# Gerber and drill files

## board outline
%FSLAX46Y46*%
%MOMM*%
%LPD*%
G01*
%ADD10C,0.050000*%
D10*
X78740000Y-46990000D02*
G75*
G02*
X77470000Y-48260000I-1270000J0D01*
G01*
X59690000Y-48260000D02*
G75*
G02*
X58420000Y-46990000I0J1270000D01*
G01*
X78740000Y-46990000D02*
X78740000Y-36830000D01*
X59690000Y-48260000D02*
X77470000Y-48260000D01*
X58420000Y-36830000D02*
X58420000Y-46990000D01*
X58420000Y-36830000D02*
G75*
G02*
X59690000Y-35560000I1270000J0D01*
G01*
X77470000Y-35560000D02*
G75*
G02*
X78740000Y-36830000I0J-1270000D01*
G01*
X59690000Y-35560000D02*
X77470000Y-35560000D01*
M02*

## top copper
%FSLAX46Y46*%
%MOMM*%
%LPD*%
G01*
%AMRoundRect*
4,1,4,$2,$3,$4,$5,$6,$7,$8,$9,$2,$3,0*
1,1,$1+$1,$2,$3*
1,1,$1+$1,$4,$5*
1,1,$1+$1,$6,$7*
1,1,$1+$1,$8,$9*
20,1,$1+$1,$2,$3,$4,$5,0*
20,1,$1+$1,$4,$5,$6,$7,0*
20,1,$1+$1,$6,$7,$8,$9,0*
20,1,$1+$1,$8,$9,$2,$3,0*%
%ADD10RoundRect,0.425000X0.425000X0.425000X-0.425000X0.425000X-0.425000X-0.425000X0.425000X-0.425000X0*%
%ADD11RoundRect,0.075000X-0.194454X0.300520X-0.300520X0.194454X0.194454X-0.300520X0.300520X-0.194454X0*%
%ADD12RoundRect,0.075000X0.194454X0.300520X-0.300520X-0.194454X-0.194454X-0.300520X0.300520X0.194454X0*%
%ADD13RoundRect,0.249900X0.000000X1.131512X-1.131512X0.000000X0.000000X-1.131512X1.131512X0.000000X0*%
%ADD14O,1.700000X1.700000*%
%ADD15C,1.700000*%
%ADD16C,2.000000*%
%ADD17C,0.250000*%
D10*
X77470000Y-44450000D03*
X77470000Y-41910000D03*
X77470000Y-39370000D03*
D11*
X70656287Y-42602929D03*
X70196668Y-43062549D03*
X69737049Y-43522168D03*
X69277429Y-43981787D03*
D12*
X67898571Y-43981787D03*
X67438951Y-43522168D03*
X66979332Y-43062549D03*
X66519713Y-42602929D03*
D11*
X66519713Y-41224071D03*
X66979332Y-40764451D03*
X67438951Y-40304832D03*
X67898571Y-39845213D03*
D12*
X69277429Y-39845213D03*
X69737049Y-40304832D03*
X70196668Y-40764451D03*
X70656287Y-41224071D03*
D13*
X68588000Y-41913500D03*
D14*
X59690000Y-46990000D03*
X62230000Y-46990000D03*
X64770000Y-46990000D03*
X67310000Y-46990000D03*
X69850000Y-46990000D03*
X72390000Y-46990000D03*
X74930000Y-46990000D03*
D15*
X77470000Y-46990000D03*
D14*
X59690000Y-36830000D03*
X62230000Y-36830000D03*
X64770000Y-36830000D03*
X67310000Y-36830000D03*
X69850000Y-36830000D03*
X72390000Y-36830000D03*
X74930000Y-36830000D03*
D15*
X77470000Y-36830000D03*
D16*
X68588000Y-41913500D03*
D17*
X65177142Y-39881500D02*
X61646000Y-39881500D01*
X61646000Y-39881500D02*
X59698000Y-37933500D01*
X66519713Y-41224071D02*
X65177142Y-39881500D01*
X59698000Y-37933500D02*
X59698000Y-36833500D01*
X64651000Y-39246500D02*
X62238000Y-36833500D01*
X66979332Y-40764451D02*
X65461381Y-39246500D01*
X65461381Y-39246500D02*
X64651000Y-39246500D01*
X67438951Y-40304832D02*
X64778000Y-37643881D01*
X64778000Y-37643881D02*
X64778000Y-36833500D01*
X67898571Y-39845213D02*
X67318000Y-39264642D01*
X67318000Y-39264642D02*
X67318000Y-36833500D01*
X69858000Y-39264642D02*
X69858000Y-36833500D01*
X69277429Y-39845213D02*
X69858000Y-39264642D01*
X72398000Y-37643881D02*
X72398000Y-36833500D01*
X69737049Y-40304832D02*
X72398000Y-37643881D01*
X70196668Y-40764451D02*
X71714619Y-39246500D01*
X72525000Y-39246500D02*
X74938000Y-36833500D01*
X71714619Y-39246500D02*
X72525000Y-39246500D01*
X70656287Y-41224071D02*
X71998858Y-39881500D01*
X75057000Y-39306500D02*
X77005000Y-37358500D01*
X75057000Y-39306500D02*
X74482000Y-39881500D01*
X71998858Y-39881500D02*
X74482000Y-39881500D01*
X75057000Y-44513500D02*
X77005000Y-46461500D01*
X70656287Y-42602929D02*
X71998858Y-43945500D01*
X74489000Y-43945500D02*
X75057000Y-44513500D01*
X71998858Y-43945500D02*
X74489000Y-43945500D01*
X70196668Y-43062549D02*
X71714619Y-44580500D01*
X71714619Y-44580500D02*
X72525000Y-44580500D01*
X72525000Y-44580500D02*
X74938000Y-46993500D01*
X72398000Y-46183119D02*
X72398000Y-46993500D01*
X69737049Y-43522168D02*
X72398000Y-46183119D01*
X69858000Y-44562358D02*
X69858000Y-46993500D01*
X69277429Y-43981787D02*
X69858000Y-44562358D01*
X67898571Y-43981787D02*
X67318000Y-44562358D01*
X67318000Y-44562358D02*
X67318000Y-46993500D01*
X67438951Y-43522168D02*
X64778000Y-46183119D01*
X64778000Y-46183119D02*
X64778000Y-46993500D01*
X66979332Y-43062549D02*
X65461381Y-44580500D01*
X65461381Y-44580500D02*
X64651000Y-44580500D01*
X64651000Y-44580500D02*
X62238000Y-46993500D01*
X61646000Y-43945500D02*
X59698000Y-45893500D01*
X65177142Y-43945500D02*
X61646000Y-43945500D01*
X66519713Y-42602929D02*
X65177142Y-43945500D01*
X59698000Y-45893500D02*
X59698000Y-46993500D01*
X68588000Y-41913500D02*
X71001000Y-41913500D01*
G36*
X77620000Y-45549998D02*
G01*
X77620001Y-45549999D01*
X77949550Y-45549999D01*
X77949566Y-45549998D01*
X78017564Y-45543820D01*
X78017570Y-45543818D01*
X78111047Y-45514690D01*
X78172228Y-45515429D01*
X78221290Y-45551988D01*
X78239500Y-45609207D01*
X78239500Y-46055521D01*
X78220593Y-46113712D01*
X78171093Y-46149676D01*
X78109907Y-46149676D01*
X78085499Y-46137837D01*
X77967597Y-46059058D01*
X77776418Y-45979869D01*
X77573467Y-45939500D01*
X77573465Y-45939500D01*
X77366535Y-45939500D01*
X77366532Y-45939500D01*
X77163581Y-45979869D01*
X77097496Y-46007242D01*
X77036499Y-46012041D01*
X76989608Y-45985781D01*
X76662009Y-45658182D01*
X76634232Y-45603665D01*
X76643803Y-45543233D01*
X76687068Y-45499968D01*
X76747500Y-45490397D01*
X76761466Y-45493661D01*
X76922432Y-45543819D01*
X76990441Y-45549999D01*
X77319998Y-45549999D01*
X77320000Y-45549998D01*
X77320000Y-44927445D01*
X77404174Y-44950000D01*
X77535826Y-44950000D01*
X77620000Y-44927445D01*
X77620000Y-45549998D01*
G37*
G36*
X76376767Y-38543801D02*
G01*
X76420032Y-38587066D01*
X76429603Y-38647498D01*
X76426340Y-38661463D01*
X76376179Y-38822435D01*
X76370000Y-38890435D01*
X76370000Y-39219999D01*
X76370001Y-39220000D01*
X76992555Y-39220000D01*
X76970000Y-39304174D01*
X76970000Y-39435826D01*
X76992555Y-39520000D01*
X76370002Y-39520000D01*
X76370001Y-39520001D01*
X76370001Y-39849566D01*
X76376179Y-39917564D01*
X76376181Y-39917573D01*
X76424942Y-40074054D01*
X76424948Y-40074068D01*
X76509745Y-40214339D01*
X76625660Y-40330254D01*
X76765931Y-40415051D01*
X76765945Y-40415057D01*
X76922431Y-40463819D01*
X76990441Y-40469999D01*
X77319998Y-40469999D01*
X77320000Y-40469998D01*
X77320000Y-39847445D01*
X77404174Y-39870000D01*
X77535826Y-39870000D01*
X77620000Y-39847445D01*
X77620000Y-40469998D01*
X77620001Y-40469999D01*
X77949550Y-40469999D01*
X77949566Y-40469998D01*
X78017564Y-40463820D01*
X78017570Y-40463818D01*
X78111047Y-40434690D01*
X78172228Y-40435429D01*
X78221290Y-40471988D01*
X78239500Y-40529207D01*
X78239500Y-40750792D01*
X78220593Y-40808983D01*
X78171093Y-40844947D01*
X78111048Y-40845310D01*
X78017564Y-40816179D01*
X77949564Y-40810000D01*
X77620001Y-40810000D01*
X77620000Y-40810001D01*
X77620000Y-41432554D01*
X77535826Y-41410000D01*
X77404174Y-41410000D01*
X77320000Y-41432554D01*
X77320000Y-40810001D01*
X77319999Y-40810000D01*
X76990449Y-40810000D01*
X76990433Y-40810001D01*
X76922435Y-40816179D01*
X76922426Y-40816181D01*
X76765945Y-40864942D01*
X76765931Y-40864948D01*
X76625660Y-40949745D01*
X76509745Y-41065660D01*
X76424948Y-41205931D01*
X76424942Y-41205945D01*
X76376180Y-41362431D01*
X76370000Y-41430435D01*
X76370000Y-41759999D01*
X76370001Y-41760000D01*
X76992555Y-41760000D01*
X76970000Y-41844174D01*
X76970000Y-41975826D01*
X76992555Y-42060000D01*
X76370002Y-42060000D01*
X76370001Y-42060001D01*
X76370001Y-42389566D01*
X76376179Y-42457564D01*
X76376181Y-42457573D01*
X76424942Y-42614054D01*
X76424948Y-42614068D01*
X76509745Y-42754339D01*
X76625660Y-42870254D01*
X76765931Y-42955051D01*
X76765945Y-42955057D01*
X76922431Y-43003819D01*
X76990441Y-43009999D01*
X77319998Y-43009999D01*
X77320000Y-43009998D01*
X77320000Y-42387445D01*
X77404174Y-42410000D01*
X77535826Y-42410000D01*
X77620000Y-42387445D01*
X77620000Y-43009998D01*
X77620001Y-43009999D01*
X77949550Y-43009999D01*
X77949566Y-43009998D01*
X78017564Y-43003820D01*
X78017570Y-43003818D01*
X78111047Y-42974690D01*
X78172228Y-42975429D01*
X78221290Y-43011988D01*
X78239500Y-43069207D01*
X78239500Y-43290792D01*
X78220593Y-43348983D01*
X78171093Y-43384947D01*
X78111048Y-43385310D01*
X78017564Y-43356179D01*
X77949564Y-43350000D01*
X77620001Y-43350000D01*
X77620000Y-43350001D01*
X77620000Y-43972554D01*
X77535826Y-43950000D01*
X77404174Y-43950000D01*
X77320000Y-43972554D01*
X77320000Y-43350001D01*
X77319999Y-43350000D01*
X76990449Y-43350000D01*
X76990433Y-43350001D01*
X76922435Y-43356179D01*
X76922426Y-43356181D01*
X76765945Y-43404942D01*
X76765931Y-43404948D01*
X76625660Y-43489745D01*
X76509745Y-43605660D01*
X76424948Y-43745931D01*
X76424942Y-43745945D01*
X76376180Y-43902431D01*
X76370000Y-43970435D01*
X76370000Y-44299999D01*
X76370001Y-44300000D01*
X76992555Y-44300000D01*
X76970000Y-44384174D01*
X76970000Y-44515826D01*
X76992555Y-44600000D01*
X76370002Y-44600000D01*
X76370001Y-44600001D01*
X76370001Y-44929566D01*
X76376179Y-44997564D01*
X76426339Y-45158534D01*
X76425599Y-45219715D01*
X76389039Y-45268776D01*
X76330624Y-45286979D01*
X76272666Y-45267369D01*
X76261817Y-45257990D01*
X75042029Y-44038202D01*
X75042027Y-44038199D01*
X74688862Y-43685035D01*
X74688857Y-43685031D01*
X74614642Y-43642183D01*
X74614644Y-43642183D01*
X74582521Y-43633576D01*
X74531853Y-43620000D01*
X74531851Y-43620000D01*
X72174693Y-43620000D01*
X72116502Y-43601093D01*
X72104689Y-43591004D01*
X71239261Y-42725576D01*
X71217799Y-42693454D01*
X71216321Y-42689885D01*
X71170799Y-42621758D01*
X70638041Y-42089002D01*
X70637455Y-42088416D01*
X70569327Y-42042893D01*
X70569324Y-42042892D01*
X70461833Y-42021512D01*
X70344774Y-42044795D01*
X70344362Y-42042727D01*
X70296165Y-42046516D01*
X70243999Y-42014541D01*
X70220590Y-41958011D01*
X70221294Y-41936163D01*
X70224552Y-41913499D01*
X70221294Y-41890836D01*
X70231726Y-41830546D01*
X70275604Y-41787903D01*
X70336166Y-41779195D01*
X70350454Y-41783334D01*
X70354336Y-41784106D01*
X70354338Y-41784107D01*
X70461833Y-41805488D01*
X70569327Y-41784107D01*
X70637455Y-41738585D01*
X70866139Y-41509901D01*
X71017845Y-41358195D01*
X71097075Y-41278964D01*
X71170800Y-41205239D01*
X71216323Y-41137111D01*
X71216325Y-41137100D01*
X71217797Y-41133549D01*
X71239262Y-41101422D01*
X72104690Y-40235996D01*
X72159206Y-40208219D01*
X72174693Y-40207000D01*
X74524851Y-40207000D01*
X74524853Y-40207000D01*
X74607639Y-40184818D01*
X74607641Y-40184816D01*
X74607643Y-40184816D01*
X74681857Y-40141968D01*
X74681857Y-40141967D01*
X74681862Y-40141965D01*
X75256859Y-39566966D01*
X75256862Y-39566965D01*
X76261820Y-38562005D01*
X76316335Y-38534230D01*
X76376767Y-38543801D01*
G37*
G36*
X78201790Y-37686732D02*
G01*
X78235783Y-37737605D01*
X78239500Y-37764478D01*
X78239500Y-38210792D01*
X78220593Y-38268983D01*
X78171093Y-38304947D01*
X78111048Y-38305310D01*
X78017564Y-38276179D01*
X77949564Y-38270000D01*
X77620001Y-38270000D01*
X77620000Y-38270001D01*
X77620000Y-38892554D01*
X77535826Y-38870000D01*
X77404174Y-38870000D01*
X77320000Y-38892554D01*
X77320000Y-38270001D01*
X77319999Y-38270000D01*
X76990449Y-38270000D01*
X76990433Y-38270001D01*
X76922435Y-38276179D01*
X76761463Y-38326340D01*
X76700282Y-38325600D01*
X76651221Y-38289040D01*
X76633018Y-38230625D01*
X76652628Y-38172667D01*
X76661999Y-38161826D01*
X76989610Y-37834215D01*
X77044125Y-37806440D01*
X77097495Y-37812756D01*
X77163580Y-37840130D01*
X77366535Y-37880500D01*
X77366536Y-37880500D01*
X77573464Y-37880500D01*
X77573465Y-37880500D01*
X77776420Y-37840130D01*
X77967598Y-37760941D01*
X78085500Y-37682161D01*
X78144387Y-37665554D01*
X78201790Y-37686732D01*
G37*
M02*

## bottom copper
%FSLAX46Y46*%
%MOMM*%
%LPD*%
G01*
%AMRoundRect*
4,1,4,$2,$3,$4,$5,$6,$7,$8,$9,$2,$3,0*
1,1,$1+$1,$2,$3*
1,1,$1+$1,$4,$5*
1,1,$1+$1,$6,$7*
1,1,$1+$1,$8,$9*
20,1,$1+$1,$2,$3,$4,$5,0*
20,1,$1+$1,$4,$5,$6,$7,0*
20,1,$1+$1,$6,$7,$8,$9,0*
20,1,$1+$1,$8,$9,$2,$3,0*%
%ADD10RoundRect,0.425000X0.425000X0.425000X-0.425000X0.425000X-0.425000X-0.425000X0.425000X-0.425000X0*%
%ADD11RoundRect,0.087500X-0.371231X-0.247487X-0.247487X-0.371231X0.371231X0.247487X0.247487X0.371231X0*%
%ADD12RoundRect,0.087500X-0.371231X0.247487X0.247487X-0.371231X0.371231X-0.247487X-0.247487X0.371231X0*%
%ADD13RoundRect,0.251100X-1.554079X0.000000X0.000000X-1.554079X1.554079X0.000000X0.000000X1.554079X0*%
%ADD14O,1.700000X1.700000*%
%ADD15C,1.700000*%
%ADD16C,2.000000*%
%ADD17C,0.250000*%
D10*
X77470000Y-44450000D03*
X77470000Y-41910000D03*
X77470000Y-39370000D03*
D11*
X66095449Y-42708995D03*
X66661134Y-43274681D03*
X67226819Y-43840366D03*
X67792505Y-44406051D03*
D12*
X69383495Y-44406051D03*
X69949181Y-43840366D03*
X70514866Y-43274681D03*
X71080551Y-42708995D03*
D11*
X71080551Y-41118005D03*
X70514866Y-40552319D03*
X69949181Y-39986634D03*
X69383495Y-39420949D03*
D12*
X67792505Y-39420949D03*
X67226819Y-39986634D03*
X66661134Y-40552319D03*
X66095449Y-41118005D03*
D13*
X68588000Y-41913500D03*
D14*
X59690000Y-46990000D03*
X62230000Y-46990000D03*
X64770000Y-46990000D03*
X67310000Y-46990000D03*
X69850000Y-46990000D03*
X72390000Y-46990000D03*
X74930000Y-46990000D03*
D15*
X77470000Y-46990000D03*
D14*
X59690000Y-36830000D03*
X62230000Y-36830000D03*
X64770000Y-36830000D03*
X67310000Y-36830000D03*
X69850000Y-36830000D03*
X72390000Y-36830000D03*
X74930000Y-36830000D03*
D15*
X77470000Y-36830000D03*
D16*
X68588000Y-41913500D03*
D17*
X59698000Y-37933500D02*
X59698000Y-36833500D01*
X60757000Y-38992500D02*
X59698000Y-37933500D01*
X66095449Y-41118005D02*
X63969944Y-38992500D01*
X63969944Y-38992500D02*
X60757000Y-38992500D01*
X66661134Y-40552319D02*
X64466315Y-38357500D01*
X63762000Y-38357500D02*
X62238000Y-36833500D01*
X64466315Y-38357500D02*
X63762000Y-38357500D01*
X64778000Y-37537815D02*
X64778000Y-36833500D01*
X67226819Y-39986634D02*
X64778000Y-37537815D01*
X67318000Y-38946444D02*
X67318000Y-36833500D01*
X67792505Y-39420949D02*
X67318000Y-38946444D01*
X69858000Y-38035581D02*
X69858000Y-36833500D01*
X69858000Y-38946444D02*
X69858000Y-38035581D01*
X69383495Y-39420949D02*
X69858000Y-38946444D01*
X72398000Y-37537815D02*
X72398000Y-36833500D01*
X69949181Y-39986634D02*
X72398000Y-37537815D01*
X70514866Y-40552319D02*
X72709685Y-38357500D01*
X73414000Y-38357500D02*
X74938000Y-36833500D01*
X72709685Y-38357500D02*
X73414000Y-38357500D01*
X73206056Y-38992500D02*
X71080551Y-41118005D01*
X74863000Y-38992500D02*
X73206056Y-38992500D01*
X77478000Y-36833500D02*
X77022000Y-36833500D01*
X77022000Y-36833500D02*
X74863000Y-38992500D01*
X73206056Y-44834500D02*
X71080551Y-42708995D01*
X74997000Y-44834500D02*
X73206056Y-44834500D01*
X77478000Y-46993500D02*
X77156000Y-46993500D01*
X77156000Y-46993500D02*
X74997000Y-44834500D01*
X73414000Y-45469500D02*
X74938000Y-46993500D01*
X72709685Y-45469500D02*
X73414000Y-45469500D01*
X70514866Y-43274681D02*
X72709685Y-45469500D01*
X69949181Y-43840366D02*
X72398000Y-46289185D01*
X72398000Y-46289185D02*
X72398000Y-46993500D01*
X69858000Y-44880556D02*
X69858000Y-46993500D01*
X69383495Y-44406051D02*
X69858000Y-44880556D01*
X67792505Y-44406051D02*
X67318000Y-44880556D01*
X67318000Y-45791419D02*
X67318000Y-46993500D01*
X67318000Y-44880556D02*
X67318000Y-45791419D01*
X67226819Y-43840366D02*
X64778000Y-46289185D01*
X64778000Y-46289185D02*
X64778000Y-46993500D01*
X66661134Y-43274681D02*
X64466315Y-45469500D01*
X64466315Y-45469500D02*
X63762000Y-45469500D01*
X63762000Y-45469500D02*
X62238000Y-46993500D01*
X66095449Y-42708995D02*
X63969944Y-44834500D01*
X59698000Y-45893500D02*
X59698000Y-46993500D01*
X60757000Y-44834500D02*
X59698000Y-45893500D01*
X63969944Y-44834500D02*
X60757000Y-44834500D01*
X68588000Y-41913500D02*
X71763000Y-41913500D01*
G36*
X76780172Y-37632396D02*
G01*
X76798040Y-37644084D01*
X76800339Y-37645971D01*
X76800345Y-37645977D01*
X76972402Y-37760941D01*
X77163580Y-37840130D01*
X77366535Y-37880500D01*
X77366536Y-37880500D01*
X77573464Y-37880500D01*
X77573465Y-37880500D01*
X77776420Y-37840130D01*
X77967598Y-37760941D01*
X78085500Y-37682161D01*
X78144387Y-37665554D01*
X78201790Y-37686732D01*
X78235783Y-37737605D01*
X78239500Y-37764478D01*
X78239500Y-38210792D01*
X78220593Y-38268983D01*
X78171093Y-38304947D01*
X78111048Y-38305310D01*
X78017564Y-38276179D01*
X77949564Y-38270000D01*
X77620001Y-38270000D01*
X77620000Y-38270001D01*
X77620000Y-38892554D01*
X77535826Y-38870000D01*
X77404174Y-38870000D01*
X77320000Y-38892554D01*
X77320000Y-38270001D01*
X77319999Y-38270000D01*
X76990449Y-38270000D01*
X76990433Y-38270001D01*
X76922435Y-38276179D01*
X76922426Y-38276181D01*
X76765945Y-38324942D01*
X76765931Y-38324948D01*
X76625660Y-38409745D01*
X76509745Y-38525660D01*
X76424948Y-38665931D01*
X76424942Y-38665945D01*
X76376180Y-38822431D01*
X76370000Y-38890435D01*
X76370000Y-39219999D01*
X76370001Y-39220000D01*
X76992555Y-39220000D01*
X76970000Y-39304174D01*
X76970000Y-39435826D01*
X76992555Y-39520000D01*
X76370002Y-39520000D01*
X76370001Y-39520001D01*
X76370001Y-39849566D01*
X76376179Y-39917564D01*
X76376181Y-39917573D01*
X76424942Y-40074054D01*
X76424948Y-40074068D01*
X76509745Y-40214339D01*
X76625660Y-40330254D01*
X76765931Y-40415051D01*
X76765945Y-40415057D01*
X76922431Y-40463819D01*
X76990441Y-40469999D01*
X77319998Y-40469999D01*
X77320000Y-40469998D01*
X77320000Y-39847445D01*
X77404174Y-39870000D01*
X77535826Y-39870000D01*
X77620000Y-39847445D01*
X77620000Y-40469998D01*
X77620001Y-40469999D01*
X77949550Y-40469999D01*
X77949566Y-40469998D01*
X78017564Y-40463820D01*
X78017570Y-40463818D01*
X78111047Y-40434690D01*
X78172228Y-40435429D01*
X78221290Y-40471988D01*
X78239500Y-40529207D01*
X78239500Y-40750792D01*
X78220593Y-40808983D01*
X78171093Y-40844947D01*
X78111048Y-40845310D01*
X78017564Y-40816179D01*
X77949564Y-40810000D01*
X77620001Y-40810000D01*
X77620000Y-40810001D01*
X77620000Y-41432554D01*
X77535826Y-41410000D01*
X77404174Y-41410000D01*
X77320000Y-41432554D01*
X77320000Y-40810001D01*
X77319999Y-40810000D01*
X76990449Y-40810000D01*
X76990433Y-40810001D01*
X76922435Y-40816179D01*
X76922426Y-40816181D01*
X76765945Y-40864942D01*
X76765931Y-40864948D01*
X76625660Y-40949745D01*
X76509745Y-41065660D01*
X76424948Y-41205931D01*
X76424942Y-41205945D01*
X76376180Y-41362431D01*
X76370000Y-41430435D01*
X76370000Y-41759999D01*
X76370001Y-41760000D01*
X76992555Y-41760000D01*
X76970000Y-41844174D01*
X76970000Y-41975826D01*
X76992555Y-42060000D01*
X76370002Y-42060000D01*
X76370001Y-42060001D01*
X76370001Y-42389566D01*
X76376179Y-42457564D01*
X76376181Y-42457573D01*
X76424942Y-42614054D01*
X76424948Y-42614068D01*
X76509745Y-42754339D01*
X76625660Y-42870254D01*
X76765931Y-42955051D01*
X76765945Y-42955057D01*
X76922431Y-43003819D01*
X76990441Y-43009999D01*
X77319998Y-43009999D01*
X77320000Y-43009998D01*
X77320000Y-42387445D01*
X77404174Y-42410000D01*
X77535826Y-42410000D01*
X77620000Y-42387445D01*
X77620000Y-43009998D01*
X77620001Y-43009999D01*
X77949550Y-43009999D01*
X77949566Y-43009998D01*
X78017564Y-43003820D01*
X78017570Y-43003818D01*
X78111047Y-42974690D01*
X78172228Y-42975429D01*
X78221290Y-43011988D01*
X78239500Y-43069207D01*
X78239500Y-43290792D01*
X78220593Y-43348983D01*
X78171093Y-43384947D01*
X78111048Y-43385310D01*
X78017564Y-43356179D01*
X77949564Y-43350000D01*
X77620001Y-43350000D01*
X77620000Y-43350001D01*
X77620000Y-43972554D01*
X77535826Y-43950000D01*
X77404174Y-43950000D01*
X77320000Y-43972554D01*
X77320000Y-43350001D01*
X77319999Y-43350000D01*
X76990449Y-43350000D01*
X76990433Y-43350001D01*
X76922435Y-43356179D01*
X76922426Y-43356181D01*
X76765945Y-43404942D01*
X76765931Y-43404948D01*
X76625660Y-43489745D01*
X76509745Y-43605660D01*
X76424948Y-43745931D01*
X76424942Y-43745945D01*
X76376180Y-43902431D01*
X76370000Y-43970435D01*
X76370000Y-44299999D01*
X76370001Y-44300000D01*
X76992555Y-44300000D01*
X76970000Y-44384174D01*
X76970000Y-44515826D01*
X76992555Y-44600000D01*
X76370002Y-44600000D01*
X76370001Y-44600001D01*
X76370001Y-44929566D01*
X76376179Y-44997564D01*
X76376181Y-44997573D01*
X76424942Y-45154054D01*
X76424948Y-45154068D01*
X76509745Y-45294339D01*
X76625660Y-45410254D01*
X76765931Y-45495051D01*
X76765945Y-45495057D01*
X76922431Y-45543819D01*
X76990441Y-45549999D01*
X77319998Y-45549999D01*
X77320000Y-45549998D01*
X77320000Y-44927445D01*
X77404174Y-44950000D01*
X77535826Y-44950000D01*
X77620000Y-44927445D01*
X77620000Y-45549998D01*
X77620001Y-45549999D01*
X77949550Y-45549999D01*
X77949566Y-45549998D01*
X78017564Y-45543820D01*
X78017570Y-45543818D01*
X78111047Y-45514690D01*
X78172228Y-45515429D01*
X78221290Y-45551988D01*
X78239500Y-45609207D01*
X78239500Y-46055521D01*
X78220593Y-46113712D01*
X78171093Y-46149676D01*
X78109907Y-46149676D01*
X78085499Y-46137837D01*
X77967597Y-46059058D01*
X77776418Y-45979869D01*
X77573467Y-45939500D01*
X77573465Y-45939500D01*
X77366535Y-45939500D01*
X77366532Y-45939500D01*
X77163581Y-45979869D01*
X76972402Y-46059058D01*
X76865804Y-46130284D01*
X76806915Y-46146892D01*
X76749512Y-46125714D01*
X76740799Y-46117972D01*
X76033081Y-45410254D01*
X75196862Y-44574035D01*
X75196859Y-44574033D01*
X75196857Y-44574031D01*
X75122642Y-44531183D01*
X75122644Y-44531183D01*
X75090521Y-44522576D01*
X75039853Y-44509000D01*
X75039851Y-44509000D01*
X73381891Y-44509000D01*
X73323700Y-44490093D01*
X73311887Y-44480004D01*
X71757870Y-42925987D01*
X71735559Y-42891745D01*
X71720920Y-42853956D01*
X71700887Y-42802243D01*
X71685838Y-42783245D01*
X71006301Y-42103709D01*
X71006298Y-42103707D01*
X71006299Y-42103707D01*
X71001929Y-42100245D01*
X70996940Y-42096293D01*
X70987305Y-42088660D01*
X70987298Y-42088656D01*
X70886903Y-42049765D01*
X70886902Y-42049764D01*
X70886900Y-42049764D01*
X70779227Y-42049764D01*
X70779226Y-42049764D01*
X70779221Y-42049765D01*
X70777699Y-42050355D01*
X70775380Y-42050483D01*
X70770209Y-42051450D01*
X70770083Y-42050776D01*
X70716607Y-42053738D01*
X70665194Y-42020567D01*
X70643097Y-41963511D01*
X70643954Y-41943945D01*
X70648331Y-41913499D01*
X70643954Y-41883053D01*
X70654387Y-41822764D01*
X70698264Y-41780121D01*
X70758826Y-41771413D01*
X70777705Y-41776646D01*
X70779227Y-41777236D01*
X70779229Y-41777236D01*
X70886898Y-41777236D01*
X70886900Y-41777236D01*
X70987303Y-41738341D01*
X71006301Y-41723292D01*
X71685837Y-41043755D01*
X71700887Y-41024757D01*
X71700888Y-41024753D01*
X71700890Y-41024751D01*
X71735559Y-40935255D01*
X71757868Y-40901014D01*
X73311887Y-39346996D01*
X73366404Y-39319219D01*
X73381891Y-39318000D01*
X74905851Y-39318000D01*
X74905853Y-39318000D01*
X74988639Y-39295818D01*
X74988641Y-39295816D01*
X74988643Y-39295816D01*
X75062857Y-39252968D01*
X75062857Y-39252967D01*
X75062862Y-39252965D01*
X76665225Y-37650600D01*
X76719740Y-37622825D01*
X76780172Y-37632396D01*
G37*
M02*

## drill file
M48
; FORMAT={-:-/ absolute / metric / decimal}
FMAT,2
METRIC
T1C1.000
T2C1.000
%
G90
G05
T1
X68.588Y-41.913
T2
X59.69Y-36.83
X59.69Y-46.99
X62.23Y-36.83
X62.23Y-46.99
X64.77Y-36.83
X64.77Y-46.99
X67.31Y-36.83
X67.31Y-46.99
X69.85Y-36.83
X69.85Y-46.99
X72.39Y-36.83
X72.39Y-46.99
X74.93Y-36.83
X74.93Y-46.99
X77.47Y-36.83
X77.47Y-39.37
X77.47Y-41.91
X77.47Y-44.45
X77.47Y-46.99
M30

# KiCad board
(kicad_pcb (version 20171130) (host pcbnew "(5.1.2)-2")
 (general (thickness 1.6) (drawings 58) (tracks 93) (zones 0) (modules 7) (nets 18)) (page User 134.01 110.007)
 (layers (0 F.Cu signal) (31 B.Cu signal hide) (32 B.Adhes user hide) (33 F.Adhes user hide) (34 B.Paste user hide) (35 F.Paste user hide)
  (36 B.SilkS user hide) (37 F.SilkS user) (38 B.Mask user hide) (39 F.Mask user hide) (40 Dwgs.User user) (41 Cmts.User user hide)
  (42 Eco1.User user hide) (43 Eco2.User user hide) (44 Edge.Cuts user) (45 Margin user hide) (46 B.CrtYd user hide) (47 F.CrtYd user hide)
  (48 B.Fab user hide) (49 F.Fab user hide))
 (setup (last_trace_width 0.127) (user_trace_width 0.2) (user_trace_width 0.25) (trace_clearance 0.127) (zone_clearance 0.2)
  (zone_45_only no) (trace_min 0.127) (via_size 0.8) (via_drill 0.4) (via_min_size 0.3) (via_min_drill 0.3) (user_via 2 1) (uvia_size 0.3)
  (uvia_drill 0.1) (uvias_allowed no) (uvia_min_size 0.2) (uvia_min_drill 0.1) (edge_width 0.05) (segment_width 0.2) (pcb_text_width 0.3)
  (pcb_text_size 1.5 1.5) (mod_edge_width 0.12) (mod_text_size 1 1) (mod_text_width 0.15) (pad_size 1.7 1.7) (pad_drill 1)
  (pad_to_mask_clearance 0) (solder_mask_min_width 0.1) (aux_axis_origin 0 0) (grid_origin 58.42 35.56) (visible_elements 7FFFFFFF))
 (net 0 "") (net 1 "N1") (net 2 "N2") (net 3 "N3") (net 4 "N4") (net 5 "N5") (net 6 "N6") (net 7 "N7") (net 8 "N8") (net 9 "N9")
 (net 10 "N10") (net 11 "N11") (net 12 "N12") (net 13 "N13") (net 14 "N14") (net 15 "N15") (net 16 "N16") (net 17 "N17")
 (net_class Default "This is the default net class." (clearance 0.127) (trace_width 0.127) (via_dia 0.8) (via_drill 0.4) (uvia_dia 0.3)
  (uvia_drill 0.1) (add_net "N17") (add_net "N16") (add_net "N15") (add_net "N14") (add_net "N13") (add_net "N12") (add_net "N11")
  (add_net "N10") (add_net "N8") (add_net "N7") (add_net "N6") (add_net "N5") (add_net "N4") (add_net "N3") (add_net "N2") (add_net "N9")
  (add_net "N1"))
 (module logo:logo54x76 (layer B.Cu) (at 62.23 41.91)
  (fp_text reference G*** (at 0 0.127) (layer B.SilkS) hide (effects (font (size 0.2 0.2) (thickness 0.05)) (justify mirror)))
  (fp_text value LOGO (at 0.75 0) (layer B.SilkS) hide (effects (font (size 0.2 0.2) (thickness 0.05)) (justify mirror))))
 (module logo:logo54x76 (layer F.Cu) (at 62.23 41.91)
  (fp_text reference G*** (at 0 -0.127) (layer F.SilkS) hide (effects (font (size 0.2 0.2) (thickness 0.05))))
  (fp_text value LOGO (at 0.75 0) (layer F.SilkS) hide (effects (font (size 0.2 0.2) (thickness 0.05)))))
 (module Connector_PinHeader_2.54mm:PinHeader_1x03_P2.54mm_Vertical (layer B.Cu) (at 77.47 39.37 180)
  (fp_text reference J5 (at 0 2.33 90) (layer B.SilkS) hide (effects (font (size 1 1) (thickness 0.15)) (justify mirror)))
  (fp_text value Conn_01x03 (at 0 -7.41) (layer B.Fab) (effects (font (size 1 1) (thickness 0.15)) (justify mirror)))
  (pad 3 thru_hole roundrect (at 0 -5.08 180) (size 1.7 1.7) (drill 1) (layers *.Cu *.Mask) (roundrect_rratio 0.25) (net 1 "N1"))
  (pad 2 thru_hole roundrect (at 0 -2.54 180) (size 1.7 1.7) (drill 1) (layers *.Cu *.Mask) (roundrect_rratio 0.25) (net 1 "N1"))
  (pad 1 thru_hole roundrect (at 0 0 180) (size 1.7 1.7) (drill 1) (layers *.Cu *.Mask) (roundrect_rratio 0.25) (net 1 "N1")))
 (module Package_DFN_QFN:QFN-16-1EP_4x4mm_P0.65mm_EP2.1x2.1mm (layer F.Cu) (at 68.588 41.9135 225)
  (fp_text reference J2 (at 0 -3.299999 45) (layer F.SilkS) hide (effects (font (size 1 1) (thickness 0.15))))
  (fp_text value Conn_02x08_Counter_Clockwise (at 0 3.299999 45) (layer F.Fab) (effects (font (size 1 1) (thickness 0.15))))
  (pad 16 smd roundrect (at -0.975 -1.95 225) (size 0.3 0.85) (layers F.Cu F.Paste F.Mask) (roundrect_rratio 0.25) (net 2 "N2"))
  (pad 15 smd roundrect (at -0.325 -1.95 225) (size 0.3 0.85) (layers F.Cu F.Paste F.Mask) (roundrect_rratio 0.25) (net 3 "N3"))
  (pad 14 smd roundrect (at 0.325 -1.95 225) (size 0.3 0.85) (layers F.Cu F.Paste F.Mask) (roundrect_rratio 0.25) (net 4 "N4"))
  (pad 13 smd roundrect (at 0.975 -1.95 225) (size 0.3 0.85) (layers F.Cu F.Paste F.Mask) (roundrect_rratio 0.25) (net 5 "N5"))
  (pad 12 smd roundrect (at 1.95 -0.975 225) (size 0.85 0.3) (layers F.Cu F.Paste F.Mask) (roundrect_rratio 0.25) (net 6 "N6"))
  (pad 11 smd roundrect (at 1.95 -0.325 225) (size 0.85 0.3) (layers F.Cu F.Paste F.Mask) (roundrect_rratio 0.25) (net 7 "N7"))
  (pad 10 smd roundrect (at 1.95 0.325 225) (size 0.85 0.3) (layers F.Cu F.Paste F.Mask) (roundrect_rratio 0.25) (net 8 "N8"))
  (pad 9 smd roundrect (at 1.95 0.975 225) (size 0.85 0.3) (layers F.Cu F.Paste F.Mask) (roundrect_rratio 0.25) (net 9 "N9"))
  (pad 8 smd roundrect (at 0.975 1.95 225) (size 0.3 0.85) (layers F.Cu F.Paste F.Mask) (roundrect_rratio 0.25) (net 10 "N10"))
  (pad 7 smd roundrect (at 0.325 1.95 225) (size 0.3 0.85) (layers F.Cu F.Paste F.Mask) (roundrect_rratio 0.25) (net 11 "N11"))
  (pad 6 smd roundrect (at -0.325 1.95 225) (size 0.3 0.85) (layers F.Cu F.Paste F.Mask) (roundrect_rratio 0.25) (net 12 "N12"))
  (pad 5 smd roundrect (at -0.975 1.95 225) (size 0.3 0.85) (layers F.Cu F.Paste F.Mask) (roundrect_rratio 0.25) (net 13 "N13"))
  (pad 4 smd roundrect (at -1.95 0.975 225) (size 0.85 0.3) (layers F.Cu F.Paste F.Mask) (roundrect_rratio 0.25) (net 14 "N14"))
  (pad 3 smd roundrect (at -1.95 0.325 225) (size 0.85 0.3) (layers F.Cu F.Paste F.Mask) (roundrect_rratio 0.25) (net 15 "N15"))
  (pad 2 smd roundrect (at -1.95 -0.325 225) (size 0.85 0.3) (layers F.Cu F.Paste F.Mask) (roundrect_rratio 0.25) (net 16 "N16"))
  (pad 1 smd roundrect (at -1.95 -0.975 225) (size 0.85 0.3) (layers F.Cu F.Paste F.Mask) (roundrect_rratio 0.25) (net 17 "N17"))
  (pad "" smd roundrect (at 0.525 0.525 225) (size 0.85 0.85) (layers F.Paste) (roundrect_rratio 0.25))
  (pad "" smd roundrect (at 0.525 -0.525 225) (size 0.85 0.85) (layers F.Paste) (roundrect_rratio 0.25))
  (pad "" smd roundrect (at -0.525 0.525 225) (size 0.85 0.85) (layers F.Paste) (roundrect_rratio 0.25))
  (pad "" smd roundrect (at -0.525 -0.525 225) (size 0.85 0.85) (layers F.Paste) (roundrect_rratio 0.25))
  (pad 17 smd roundrect (at 0 0 225) (size 2.1 2.1) (layers F.Cu F.Mask) (roundrect_rratio 0.119) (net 1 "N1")))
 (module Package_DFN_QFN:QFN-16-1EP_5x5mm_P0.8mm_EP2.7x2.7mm (layer B.Cu) (at 68.588 41.9135 315)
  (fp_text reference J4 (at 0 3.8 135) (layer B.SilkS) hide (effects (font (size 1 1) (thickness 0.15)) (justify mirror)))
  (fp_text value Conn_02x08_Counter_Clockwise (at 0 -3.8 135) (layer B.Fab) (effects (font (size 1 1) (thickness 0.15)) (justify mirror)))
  (pad 16 smd roundrect (at -1.2 2.325 315) (size 0.35 1.05) (layers B.Cu B.Paste B.Mask) (roundrect_rratio 0.25) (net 9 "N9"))
  (pad 15 smd roundrect (at -0.4 2.325 315) (size 0.35 1.05) (layers B.Cu B.Paste B.Mask) (roundrect_rratio 0.25) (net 8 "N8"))
  (pad 14 smd roundrect (at 0.4 2.325 315) (size 0.35 1.05) (layers B.Cu B.Paste B.Mask) (roundrect_rratio 0.25) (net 7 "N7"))
  (pad 13 smd roundrect (at 1.2 2.325 315) (size 0.35 1.05) (layers B.Cu B.Paste B.Mask) (roundrect_rratio 0.25) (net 6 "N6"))
  (pad 12 smd roundrect (at 2.325 1.2 315) (size 1.05 0.35) (layers B.Cu B.Paste B.Mask) (roundrect_rratio 0.25) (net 5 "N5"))
  (pad 11 smd roundrect (at 2.325 0.4 315) (size 1.05 0.35) (layers B.Cu B.Paste B.Mask) (roundrect_rratio 0.25) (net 4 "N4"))
  (pad 10 smd roundrect (at 2.325 -0.4 315) (size 1.05 0.35) (layers B.Cu B.Paste B.Mask) (roundrect_rratio 0.25) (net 3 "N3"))
  (pad 9 smd roundrect (at 2.325 -1.2 315) (size 1.05 0.35) (layers B.Cu B.Paste B.Mask) (roundrect_rratio 0.25) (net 2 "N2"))
  (pad 8 smd roundrect (at 1.2 -2.325 315) (size 0.35 1.05) (layers B.Cu B.Paste B.Mask) (roundrect_rratio 0.25) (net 17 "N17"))
  (pad 7 smd roundrect (at 0.4 -2.325 315) (size 0.35 1.05) (layers B.Cu B.Paste B.Mask) (roundrect_rratio 0.25) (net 16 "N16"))
  (pad 6 smd roundrect (at -0.4 -2.325 315) (size 0.35 1.05) (layers B.Cu B.Paste B.Mask) (roundrect_rratio 0.25) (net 15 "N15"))
  (pad 5 smd roundrect (at -1.2 -2.325 315) (size 0.35 1.05) (layers B.Cu B.Paste B.Mask) (roundrect_rratio 0.25) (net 14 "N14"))
  (pad 4 smd roundrect (at -2.325 -1.2 315) (size 1.05 0.35) (layers B.Cu B.Paste B.Mask) (roundrect_rratio 0.25) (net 13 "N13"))
  (pad 3 smd roundrect (at -2.325 -0.4 315) (size 1.05 0.35) (layers B.Cu B.Paste B.Mask) (roundrect_rratio 0.25) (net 12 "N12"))
  (pad 2 smd roundrect (at -2.325 0.4 315) (size 1.05 0.35) (layers B.Cu B.Paste B.Mask) (roundrect_rratio 0.25) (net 11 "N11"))
  (pad 1 smd roundrect (at -2.325 1.2 315) (size 1.05 0.35) (layers B.Cu B.Paste B.Mask) (roundrect_rratio 0.25) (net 10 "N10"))
  (pad "" smd roundrect (at 0.675 -0.675 315) (size 1.09 1.09) (layers B.Paste) (roundrect_rratio 0.229358))
  (pad "" smd roundrect (at 0.675 0.675 315) (size 1.09 1.09) (layers B.Paste) (roundrect_rratio 0.229358))
  (pad "" smd roundrect (at -0.675 -0.675 315) (size 1.09 1.09) (layers B.Paste) (roundrect_rratio 0.229358))
  (pad "" smd roundrect (at -0.675 0.675 315) (size 1.09 1.09) (layers B.Paste) (roundrect_rratio 0.229358))
  (pad 17 smd roundrect (at 0 0 315) (size 2.7 2.7) (layers B.Cu B.Mask) (roundrect_rratio 0.09300000000000001) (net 1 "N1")))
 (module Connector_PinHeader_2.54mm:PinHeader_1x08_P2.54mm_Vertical (layer F.Cu) (at 77.47 46.99 270)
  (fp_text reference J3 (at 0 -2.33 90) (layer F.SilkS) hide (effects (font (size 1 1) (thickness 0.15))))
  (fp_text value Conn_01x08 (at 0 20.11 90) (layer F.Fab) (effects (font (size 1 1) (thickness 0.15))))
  (pad 8 thru_hole oval (at 0 17.78 270) (size 1.7 1.7) (drill 1) (layers *.Cu *.Mask) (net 9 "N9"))
  (pad 7 thru_hole oval (at 0 15.24 270) (size 1.7 1.7) (drill 1) (layers *.Cu *.Mask) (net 8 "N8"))
  (pad 6 thru_hole oval (at 0 12.7 270) (size 1.7 1.7) (drill 1) (layers *.Cu *.Mask) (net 7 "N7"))
  (pad 5 thru_hole oval (at 0 10.16 270) (size 1.7 1.7) (drill 1) (layers *.Cu *.Mask) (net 6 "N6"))
  (pad 4 thru_hole oval (at 0 7.62 270) (size 1.7 1.7) (drill 1) (layers *.Cu *.Mask) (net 5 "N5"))
  (pad 3 thru_hole oval (at 0 5.08 270) (size 1.7 1.7) (drill 1) (layers *.Cu *.Mask) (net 4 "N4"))
  (pad 2 thru_hole oval (at 0 2.54 270) (size 1.7 1.7) (drill 1) (layers *.Cu *.Mask) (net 3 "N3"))
  (pad 1 thru_hole circle (at 0 0 270) (size 1.7 1.7) (drill 1) (layers *.Cu *.Mask) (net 2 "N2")))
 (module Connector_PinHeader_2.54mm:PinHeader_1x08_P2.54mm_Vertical (layer F.Cu) (at 77.47 36.83 270)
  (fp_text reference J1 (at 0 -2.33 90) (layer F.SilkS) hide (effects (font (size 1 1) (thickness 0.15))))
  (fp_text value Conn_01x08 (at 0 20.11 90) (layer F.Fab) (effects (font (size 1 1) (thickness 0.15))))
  (pad 8 thru_hole oval (at 0 17.78 270) (size 1.7 1.7) (drill 1) (layers *.Cu *.Mask) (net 10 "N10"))
  (pad 7 thru_hole oval (at 0 15.24 270) (size 1.7 1.7) (drill 1) (layers *.Cu *.Mask) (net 11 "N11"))
  (pad 6 thru_hole oval (at 0 12.7 270) (size 1.7 1.7) (drill 1) (layers *.Cu *.Mask) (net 12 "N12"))
  (pad 5 thru_hole oval (at 0 10.16 270) (size 1.7 1.7) (drill 1) (layers *.Cu *.Mask) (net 13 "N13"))
  (pad 4 thru_hole oval (at 0 7.62 270) (size 1.7 1.7) (drill 1) (layers *.Cu *.Mask) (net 14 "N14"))
  (pad 3 thru_hole oval (at 0 5.08 270) (size 1.7 1.7) (drill 1) (layers *.Cu *.Mask) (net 15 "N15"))
  (pad 2 thru_hole oval (at 0 2.54 270) (size 1.7 1.7) (drill 1) (layers *.Cu *.Mask) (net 16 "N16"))
  (pad 1 thru_hole circle (at 0 0 270) (size 1.7 1.7) (drill 1) (layers *.Cu *.Mask) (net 17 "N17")))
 (gr_arc (start 77.47 46.99) (end 77.47 48.26) (angle -90) (layer Edge.Cuts) (width 0.05))
 (gr_arc (start 59.69 46.99) (end 58.42 46.99) (angle -90) (layer Edge.Cuts) (width 0.05))
 (gr_line (start 78.74 46.99) (end 78.74 36.83) (layer Edge.Cuts) (width 0.05))
 (gr_line (start 59.69 48.26) (end 77.47 48.26) (layer Edge.Cuts) (width 0.05))
 (gr_line (start 58.42 36.83) (end 58.42 46.99) (layer Edge.Cuts) (width 0.05))
 (gr_arc (start 59.69 36.83) (end 59.69 35.56) (angle -90) (layer Edge.Cuts) (width 0.05))
 (gr_arc (start 77.47 36.83) (end 78.74 36.83) (angle -90) (layer Edge.Cuts) (width 0.05))
 (gr_line (start 59.69 35.56) (end 77.47 35.56) (layer Edge.Cuts) (width 0.05))
 (segment (start 65.177142 39.8815) (end 61.646 39.8815) (width 0.25) (layer F.Cu) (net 10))
 (segment (start 61.646 39.8815) (end 59.698 37.9335) (width 0.25) (layer F.Cu) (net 10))
 (segment (start 66.519713 41.224071) (end 65.177142 39.8815) (width 0.25) (layer F.Cu) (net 10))
 (segment (start 59.698 37.9335) (end 59.698 36.8335) (width 0.25) (layer F.Cu) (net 10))
 (segment (start 59.698 37.9335) (end 59.698 36.8335) (width 0.25) (layer B.Cu) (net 10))
 (segment (start 60.757 38.9925) (end 59.698 37.9335) (width 0.25) (layer B.Cu) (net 10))
 (segment (start 66.095449 41.118005) (end 63.969944 38.9925) (width 0.25) (layer B.Cu) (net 10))
 (segment (start 63.969944 38.9925) (end 60.757 38.9925) (width 0.25) (layer B.Cu) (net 10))
 (segment (start 66.661134 40.552319) (end 64.466315 38.3575) (width 0.25) (layer B.Cu) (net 11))
 (segment (start 63.762 38.3575) (end 62.238 36.8335) (width 0.25) (layer B.Cu) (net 11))
 (segment (start 64.466315 38.3575) (end 63.762 38.3575) (width 0.25) (layer B.Cu) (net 11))
 (segment (start 64.651 39.2465) (end 62.238 36.8335) (width 0.25) (layer F.Cu) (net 11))
 (segment (start 66.979332 40.764451) (end 65.461381 39.2465) (width 0.25) (layer F.Cu) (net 11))
 (segment (start 65.461381 39.2465) (end 64.651 39.2465) (width 0.25) (layer F.Cu) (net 11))
 (segment (start 64.778 37.537815) (end 64.778 36.8335) (width 0.25) (layer B.Cu) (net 12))
 (segment (start 67.226819 39.986634) (end 64.778 37.537815) (width 0.25) (layer B.Cu) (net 12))
 (segment (start 67.438951 40.304832) (end 64.778 37.643881) (width 0.25) (layer F.Cu) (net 12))
 (segment (start 64.778 37.643881) (end 64.778 36.8335) (width 0.25) (layer F.Cu) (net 12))
 (segment (start 67.898571 39.845213) (end 67.318 39.264642) (width 0.25) (layer F.Cu) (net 13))
 (segment (start 67.318 39.264642) (end 67.318 36.8335) (width 0.25) (layer F.Cu) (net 13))
 (segment (start 67.318 38.946444) (end 67.318 36.8335) (width 0.25) (layer B.Cu) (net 13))
 (segment (start 67.792505 39.420949) (end 67.318 38.946444) (width 0.25) (layer B.Cu) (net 13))
 (segment (start 69.858 39.264642) (end 69.858 36.8335) (width 0.25) (layer F.Cu) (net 14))
 (segment (start 69.277429 39.845213) (end 69.858 39.264642) (width 0.25) (layer F.Cu) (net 14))
 (segment (start 69.858 38.035581) (end 69.858 36.8335) (width 0.25) (layer B.Cu) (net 14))
 (segment (start 69.858 38.946444) (end 69.858 38.035581) (width 0.25) (layer B.Cu) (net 14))
 (segment (start 69.383495 39.420949) (end 69.858 38.946444) (width 0.25) (layer B.Cu) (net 14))
 (segment (start 72.398 37.643881) (end 72.398 36.8335) (width 0.25) (layer F.Cu) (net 15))
 (segment (start 69.737049 40.304832) (end 72.398 37.643881) (width 0.25) (layer F.Cu) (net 15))
 (segment (start 72.398 37.537815) (end 72.398 36.8335) (width 0.25) (layer B.Cu) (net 15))
 (segment (start 69.949181 39.986634) (end 72.398 37.537815) (width 0.25) (layer B.Cu) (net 15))
 (segment (start 70.196668 40.764451) (end 71.714619 39.2465) (width 0.25) (layer F.Cu) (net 16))
 (segment (start 72.525 39.2465) (end 74.938 36.8335) (width 0.25) (layer F.Cu) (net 16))
 (segment (start 71.714619 39.2465) (end 72.525 39.2465) (width 0.25) (layer F.Cu) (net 16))
 (segment (start 70.514866 40.552319) (end 72.709685 38.3575) (width 0.25) (layer B.Cu) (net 16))
 (segment (start 73.414 38.3575) (end 74.938 36.8335) (width 0.25) (layer B.Cu) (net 16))
 (segment (start 72.709685 38.3575) (end 73.414 38.3575) (width 0.25) (layer B.Cu) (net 16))
 (segment (start 70.656287 41.224071) (end 71.998858 39.8815) (width 0.25) (layer F.Cu) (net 17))
 (segment (start 75.057 39.3065) (end 77.005 37.3585) (width 0.25) (layer F.Cu) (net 17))
 (segment (start 73.206056 38.9925) (end 71.080551 41.118005) (width 0.25) (layer B.Cu) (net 17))
 (segment (start 74.863 38.9925) (end 73.206056 38.9925) (width 0.25) (layer B.Cu) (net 17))
 (segment (start 77.478 36.8335) (end 77.022 36.8335) (width 0.25) (layer B.Cu) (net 17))
 (segment (start 77.022 36.8335) (end 74.863 38.9925) (width 0.25) (layer B.Cu) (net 17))
 (segment (start 75.057 39.3065) (end 74.482 39.8815) (width 0.25) (layer F.Cu) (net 17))
 (segment (start 71.998858 39.8815) (end 74.482 39.8815) (width 0.25) (layer F.Cu) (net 17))
 (segment (start 73.206056 44.8345) (end 71.080551 42.708995) (width 0.25) (layer B.Cu) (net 2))
 (segment (start 74.997 44.8345) (end 73.206056 44.8345) (width 0.25) (layer B.Cu) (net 2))
 (segment (start 77.478 46.9935) (end 77.156 46.9935) (width 0.25) (layer B.Cu) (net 2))
 (segment (start 77.156 46.9935) (end 74.997 44.8345) (width 0.25) (layer B.Cu) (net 2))
 (segment (start 75.057 44.5135) (end 77.005 46.4615) (width 0.25) (layer F.Cu) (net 2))
 (segment (start 70.656287 42.602929) (end 71.998858 43.9455) (width 0.25) (layer F.Cu) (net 2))
 (segment (start 74.489 43.9455) (end 75.057 44.5135) (width 0.25) (layer F.Cu) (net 2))
 (segment (start 71.998858 43.9455) (end 74.489 43.9455) (width 0.25) (layer F.Cu) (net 2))
 (segment (start 73.414 45.4695) (end 74.938 46.9935) (width 0.25) (layer B.Cu) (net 3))
 (segment (start 72.709685 45.4695) (end 73.414 45.4695) (width 0.25) (layer B.Cu) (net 3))
 (segment (start 70.514866 43.274681) (end 72.709685 45.4695) (width 0.25) (layer B.Cu) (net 3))
 (segment (start 70.196668 43.062549) (end 71.714619 44.5805) (width 0.25) (layer F.Cu) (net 3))
 (segment (start 71.714619 44.5805) (end 72.525 44.5805) (width 0.25) (layer F.Cu) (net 3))
 (segment (start 72.525 44.5805) (end 74.938 46.9935) (width 0.25) (layer F.Cu) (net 3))
 (segment (start 69.949181 43.840366) (end 72.398 46.289185) (width 0.25) (layer B.Cu) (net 4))
 (segment (start 72.398 46.289185) (end 72.398 46.9935) (width 0.25) (layer B.Cu) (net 4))
 (segment (start 72.398 46.183119) (end 72.398 46.9935) (width 0.25) (layer F.Cu) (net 4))
 (segment (start 69.737049 43.522168) (end 72.398 46.183119) (width 0.25) (layer F.Cu) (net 4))
 (segment (start 69.858 44.562358) (end 69.858 46.9935) (width 0.25) (layer F.Cu) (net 5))
 (segment (start 69.277429 43.981787) (end 69.858 44.562358) (width 0.25) (layer F.Cu) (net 5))
 (segment (start 69.858 44.880556) (end 69.858 46.9935) (width 0.25) (layer B.Cu) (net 5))
 (segment (start 69.383495 44.406051) (end 69.858 44.880556) (width 0.25) (layer B.Cu) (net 5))
 (segment (start 67.792505 44.406051) (end 67.318 44.880556) (width 0.25) (layer B.Cu) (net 6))
 (segment (start 67.318 45.791419) (end 67.318 46.9935) (width 0.25) (layer B.Cu) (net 6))
 (segment (start 67.318 44.880556) (end 67.318 45.791419) (width 0.25) (layer B.Cu) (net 6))
 (segment (start 67.898571 43.981787) (end 67.318 44.562358) (width 0.25) (layer F.Cu) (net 6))
 (segment (start 67.318 44.562358) (end 67.318 46.9935) (width 0.25) (layer F.Cu) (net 6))
 (segment (start 67.226819 43.840366) (end 64.778 46.289185) (width 0.25) (layer B.Cu) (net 7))
 (segment (start 64.778 46.289185) (end 64.778 46.9935) (width 0.25) (layer B.Cu) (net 7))
 (segment (start 67.438951 43.522168) (end 64.778 46.183119) (width 0.25) (layer F.Cu) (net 7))
 (segment (start 64.778 46.183119) (end 64.778 46.9935) (width 0.25) (layer F.Cu) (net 7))
 (segment (start 66.661134 43.274681) (end 64.466315 45.4695) (width 0.25) (layer B.Cu) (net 8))
 (segment (start 64.466315 45.4695) (end 63.762 45.4695) (width 0.25) (layer B.Cu) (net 8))
 (segment (start 63.762 45.4695) (end 62.238 46.9935) (width 0.25) (layer B.Cu) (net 8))
 (segment (start 66.979332 43.062549) (end 65.461381 44.5805) (width 0.25) (layer F.Cu) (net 8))
 (segment (start 65.461381 44.5805) (end 64.651 44.5805) (width 0.25) (layer F.Cu) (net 8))
 (segment (start 64.651 44.5805) (end 62.238 46.9935) (width 0.25) (layer F.Cu) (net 8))
 (segment (start 66.095449 42.708995) (end 63.969944 44.8345) (width 0.25) (layer B.Cu) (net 9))
 (segment (start 59.698 45.8935) (end 59.698 46.9935) (width 0.25) (layer B.Cu) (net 9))
 (segment (start 60.757 44.8345) (end 59.698 45.8935) (width 0.25) (layer B.Cu) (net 9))
 (segment (start 63.969944 44.8345) (end 60.757 44.8345) (width 0.25) (layer B.Cu) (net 9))
 (segment (start 61.646 43.9455) (end 59.698 45.8935) (width 0.25) (layer F.Cu) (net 9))
 (segment (start 65.177142 43.9455) (end 61.646 43.9455) (width 0.25) (layer F.Cu) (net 9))
 (segment (start 66.519713 42.602929) (end 65.177142 43.9455) (width 0.25) (layer F.Cu) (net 9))
 (segment (start 59.698 45.8935) (end 59.698 46.9935) (width 0.25) (layer F.Cu) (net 9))
 (via (at 68.588 41.9135) (size 2) (drill 1) (layers F.Cu B.Cu) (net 1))
 (segment (start 68.588 41.9135) (end 71.763 41.9135) (width 0.25) (layer B.Cu) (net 1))
 (segment (start 68.588 41.9135) (end 71.001 41.9135) (width 0.25) (layer F.Cu) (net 1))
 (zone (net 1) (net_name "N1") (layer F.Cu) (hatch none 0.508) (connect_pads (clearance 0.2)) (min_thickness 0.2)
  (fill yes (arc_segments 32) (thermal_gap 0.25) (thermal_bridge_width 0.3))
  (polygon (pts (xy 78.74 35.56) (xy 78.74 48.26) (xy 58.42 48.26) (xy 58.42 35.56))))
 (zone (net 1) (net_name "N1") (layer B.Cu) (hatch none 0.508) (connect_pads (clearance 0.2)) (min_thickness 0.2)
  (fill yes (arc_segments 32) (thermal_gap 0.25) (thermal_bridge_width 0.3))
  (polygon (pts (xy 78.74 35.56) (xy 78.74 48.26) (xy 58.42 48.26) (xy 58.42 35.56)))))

